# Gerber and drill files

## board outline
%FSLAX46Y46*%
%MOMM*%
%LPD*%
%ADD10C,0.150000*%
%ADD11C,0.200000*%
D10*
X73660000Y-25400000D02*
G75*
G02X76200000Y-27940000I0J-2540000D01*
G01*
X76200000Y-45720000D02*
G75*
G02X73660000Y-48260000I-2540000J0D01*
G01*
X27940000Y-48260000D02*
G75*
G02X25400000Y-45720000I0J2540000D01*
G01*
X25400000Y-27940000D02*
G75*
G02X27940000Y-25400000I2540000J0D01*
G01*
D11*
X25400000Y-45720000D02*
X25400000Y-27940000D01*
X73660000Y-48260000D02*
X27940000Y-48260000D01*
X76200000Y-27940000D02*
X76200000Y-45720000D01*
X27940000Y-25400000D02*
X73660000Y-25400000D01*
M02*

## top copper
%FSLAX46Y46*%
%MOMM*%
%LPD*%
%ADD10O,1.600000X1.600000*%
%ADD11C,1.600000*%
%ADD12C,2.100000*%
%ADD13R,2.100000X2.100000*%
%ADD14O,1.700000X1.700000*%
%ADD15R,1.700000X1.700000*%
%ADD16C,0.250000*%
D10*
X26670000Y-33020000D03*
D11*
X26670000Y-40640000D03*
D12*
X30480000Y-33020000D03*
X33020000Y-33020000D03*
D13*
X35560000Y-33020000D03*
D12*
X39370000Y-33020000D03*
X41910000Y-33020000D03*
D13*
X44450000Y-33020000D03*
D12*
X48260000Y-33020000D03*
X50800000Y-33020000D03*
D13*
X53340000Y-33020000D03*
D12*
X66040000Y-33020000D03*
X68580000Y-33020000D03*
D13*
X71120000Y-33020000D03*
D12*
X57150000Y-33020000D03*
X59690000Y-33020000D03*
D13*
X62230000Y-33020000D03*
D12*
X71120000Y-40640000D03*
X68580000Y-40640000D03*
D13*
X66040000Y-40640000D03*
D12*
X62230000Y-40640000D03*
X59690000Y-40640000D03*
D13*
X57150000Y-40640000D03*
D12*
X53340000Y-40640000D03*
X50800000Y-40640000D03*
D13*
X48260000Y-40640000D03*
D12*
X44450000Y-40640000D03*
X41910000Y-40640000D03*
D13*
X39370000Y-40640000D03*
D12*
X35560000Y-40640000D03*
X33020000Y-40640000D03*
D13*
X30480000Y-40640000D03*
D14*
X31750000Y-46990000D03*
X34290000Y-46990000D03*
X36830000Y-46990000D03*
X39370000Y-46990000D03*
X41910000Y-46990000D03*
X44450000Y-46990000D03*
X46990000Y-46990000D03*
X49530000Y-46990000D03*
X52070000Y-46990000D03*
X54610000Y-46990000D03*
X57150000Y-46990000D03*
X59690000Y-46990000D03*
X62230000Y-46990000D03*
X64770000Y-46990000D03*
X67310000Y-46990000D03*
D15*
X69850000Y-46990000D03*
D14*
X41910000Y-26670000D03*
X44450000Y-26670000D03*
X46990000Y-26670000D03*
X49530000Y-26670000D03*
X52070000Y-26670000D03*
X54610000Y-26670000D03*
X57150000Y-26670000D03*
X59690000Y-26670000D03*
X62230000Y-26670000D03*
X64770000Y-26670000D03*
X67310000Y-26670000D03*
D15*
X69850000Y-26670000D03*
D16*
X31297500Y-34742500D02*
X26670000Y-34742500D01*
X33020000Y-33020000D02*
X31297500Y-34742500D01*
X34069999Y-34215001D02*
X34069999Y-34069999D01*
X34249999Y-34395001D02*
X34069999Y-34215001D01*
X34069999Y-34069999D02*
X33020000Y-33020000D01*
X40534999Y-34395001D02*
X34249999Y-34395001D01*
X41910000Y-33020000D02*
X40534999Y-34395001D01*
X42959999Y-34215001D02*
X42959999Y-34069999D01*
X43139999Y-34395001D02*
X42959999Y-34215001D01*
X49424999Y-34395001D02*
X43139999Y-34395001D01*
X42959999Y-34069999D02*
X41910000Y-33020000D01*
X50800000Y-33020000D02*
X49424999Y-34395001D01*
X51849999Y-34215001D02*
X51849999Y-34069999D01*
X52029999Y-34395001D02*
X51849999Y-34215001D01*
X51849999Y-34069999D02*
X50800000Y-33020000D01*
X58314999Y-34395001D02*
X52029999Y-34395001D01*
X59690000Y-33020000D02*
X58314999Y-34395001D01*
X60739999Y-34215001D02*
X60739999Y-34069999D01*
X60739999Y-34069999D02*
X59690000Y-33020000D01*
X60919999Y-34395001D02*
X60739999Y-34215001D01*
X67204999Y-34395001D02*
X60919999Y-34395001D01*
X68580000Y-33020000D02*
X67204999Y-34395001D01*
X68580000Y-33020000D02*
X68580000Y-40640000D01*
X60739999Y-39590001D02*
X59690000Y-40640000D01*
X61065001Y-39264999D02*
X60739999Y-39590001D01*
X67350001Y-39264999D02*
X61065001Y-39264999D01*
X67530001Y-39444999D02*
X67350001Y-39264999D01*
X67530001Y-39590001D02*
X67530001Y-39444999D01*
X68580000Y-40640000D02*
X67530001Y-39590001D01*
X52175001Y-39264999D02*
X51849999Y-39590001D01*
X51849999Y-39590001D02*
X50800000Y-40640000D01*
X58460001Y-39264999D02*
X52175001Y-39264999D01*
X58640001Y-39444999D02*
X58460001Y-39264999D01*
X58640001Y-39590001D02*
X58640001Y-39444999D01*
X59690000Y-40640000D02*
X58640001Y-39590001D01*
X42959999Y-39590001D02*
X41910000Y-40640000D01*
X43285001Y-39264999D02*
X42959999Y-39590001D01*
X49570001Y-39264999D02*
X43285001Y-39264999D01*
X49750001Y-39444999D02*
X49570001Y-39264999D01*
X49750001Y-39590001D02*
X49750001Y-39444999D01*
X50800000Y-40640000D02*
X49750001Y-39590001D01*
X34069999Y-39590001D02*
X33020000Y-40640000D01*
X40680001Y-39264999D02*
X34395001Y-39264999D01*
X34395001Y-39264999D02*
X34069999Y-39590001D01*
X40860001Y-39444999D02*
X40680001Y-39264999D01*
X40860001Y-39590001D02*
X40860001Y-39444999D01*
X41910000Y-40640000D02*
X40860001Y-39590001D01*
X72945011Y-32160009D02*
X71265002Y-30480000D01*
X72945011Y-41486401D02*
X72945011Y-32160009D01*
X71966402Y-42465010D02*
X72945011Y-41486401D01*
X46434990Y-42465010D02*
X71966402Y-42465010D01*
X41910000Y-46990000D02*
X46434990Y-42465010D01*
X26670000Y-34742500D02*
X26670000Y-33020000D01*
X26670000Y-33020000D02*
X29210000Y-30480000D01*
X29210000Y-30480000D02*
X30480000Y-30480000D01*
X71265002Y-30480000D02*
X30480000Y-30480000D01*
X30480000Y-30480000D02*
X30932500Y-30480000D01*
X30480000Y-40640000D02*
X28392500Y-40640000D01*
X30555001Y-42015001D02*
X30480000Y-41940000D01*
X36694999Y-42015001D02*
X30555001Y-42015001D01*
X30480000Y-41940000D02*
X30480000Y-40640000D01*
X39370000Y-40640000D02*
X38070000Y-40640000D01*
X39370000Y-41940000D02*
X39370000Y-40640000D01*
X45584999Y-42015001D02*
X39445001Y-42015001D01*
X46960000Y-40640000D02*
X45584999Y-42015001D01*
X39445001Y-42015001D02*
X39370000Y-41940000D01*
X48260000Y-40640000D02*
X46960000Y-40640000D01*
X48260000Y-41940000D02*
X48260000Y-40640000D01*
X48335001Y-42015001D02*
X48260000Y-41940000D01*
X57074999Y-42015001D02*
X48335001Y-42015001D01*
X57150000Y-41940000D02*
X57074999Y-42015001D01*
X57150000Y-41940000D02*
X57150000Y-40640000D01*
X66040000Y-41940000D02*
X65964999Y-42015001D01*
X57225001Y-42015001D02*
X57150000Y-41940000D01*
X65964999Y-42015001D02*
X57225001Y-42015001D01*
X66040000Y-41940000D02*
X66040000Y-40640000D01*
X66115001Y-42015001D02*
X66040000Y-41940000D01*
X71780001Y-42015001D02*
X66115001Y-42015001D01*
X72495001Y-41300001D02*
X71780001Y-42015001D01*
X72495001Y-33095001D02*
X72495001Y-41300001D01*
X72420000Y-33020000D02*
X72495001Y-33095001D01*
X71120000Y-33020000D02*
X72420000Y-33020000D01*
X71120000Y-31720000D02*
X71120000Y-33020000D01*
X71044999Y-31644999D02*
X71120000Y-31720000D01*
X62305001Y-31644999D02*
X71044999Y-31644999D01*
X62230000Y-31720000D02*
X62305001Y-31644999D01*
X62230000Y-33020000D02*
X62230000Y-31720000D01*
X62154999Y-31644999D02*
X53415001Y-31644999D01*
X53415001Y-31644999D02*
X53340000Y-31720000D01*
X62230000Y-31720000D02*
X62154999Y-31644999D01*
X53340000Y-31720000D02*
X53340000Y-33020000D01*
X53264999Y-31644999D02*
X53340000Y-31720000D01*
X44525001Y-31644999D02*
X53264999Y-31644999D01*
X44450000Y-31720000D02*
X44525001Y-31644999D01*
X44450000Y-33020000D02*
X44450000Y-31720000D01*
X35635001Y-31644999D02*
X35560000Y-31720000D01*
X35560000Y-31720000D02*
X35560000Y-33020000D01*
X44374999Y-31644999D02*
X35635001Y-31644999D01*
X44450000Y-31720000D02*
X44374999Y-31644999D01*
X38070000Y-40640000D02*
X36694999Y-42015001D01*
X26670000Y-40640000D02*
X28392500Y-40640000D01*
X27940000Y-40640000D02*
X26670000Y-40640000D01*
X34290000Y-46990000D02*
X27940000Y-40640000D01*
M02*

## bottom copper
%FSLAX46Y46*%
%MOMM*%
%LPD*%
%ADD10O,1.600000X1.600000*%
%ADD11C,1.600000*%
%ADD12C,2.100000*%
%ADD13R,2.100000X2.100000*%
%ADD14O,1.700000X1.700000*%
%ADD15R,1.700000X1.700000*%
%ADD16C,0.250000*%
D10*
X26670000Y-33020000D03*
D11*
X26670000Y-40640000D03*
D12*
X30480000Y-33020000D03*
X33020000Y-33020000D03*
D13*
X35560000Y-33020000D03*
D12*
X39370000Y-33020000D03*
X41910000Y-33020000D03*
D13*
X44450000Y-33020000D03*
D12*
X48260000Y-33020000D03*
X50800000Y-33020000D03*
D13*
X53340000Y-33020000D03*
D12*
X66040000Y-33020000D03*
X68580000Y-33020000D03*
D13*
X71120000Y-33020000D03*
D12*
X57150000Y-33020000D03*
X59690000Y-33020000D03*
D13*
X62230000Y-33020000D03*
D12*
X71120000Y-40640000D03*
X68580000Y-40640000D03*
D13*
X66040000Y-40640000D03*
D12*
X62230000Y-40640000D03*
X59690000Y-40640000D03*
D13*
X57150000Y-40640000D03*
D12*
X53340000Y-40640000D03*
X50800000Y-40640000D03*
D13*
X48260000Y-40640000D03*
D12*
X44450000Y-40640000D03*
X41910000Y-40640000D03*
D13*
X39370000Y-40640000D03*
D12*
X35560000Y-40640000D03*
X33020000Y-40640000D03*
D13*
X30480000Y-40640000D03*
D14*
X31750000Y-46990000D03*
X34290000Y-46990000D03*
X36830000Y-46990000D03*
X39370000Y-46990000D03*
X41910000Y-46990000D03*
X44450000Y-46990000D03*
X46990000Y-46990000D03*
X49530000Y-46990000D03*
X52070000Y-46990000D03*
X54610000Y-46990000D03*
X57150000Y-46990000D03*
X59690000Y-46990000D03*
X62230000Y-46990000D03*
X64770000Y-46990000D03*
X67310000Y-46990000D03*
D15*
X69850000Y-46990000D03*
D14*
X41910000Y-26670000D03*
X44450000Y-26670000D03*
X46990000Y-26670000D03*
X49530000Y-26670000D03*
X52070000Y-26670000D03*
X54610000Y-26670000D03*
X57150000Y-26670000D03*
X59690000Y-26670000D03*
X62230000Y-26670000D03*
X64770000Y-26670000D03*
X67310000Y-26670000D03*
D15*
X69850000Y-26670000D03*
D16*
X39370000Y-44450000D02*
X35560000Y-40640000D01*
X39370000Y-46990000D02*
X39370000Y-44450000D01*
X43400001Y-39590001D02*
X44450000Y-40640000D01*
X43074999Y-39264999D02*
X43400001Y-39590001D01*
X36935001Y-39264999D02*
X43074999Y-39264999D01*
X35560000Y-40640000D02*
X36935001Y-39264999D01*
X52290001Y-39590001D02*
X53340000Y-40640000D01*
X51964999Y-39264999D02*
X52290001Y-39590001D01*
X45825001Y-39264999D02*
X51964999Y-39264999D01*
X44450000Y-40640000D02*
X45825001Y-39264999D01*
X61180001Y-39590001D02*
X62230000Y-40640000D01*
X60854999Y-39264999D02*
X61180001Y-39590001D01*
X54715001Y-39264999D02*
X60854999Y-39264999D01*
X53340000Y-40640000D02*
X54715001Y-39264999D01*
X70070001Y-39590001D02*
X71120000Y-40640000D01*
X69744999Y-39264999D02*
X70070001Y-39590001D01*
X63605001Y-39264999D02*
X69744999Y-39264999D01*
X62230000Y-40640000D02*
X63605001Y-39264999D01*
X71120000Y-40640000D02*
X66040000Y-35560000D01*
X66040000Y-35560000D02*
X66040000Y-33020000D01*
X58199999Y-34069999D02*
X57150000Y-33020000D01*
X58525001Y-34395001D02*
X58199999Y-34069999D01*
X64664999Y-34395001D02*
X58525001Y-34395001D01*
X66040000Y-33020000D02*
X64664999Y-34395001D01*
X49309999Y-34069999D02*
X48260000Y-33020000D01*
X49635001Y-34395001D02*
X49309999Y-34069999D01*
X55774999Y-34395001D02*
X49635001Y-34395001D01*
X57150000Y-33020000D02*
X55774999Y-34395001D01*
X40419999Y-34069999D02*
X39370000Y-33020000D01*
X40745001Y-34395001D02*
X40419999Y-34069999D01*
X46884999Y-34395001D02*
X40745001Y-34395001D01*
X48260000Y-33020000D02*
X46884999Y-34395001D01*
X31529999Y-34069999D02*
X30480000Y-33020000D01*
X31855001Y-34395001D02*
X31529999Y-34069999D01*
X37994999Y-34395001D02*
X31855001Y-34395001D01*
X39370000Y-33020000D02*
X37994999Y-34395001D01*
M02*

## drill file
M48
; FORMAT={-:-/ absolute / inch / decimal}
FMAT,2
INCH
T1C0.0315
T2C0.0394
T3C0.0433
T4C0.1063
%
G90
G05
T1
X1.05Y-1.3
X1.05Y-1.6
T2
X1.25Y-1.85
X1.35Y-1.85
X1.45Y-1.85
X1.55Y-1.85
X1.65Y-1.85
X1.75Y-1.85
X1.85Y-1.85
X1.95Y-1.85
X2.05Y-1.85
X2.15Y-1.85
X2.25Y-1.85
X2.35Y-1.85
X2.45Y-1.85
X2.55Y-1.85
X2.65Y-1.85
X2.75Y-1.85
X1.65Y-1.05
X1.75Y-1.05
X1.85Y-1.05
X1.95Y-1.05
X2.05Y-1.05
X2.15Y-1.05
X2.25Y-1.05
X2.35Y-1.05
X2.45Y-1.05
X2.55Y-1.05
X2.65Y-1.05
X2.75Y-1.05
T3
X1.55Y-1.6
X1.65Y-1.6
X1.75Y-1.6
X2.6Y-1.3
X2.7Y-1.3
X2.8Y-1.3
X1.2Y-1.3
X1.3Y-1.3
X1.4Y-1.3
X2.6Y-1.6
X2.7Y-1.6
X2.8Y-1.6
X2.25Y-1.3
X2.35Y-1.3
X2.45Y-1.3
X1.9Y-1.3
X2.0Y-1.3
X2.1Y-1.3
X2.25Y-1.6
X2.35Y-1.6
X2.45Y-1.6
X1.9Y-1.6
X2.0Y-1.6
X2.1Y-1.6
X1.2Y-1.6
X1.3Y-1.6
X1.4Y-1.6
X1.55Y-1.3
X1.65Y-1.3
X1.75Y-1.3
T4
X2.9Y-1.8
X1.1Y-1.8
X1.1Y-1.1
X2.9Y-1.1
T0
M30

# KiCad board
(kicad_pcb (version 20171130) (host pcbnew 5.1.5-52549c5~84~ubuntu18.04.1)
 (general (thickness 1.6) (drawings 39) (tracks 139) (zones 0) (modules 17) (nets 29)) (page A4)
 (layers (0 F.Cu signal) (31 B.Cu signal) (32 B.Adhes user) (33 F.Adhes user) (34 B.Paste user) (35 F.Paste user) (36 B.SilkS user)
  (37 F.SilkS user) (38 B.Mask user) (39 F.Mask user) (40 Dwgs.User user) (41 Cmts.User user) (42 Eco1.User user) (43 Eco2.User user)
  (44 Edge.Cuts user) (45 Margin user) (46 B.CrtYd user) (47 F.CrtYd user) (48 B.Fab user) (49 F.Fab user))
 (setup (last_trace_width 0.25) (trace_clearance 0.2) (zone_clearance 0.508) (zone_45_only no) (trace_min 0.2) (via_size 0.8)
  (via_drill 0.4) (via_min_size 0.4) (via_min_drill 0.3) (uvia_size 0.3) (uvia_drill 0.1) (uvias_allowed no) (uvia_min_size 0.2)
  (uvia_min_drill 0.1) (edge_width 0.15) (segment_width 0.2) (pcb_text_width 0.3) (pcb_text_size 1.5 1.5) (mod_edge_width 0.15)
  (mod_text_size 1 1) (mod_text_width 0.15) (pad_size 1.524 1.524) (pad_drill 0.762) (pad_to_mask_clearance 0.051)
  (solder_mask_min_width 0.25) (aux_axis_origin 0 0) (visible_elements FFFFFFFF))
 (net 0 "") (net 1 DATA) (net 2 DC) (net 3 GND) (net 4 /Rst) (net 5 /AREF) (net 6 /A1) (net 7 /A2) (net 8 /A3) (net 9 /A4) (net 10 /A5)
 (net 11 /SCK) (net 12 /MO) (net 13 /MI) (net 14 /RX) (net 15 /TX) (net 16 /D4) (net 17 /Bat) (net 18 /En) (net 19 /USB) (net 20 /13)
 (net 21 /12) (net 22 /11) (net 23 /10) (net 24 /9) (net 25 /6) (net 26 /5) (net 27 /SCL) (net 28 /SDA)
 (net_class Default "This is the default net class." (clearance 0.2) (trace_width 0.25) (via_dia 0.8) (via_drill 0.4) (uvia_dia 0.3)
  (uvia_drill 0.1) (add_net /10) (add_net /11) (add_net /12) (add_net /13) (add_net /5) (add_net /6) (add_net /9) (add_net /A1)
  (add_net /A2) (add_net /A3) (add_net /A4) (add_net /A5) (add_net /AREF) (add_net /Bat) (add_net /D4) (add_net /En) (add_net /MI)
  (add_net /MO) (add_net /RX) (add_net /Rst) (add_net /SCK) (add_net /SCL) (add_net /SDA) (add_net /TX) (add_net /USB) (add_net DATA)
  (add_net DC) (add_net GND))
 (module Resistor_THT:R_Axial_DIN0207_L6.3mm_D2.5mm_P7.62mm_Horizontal (layer F.Cu) (at 26.67 40.64 90)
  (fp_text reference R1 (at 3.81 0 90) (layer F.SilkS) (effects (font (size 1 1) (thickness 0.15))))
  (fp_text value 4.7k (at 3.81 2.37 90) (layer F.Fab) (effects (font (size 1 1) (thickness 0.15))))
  (pad 2 thru_hole oval (at 7.62 0 90) (size 1.6 1.6) (drill 0.8) (layers *.Cu *.Mask) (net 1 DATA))
  (pad 1 thru_hole circle (at 0 0 90) (size 1.6 1.6) (drill 0.8) (layers *.Cu *.Mask) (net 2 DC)))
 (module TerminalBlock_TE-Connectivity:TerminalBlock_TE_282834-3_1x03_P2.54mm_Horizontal (layer F.Cu) (at 35.56 33.02 180)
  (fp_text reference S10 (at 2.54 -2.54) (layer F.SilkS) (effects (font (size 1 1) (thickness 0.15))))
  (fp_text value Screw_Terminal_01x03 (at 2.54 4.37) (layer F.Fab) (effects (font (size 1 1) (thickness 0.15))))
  (pad 3 thru_hole circle (at 5.08 0 180) (size 2.1 2.1) (drill 1.1) (layers *.Cu *.Mask) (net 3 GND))
  (pad 2 thru_hole circle (at 2.54 0 180) (size 2.1 2.1) (drill 1.1) (layers *.Cu *.Mask) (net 1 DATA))
  (pad 1 thru_hole rect (at 0 0 180) (size 2.1 2.1) (drill 1.1) (layers *.Cu *.Mask) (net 2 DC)))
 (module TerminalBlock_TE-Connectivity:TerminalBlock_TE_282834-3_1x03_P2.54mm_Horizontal (layer F.Cu) (at 44.45 33.02 180)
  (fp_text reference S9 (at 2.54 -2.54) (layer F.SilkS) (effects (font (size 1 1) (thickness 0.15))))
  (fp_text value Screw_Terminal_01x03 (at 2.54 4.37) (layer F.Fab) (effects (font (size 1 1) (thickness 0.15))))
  (pad 3 thru_hole circle (at 5.08 0 180) (size 2.1 2.1) (drill 1.1) (layers *.Cu *.Mask) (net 3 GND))
  (pad 2 thru_hole circle (at 2.54 0 180) (size 2.1 2.1) (drill 1.1) (layers *.Cu *.Mask) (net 1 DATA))
  (pad 1 thru_hole rect (at 0 0 180) (size 2.1 2.1) (drill 1.1) (layers *.Cu *.Mask) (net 2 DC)))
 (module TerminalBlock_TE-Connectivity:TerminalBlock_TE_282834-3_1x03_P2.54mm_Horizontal (layer F.Cu) (at 53.34 33.02 180)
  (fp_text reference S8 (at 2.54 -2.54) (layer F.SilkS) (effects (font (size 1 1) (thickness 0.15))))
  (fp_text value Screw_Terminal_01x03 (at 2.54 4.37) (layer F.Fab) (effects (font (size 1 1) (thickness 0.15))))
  (pad 3 thru_hole circle (at 5.08 0 180) (size 2.1 2.1) (drill 1.1) (layers *.Cu *.Mask) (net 3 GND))
  (pad 2 thru_hole circle (at 2.54 0 180) (size 2.1 2.1) (drill 1.1) (layers *.Cu *.Mask) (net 1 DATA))
  (pad 1 thru_hole rect (at 0 0 180) (size 2.1 2.1) (drill 1.1) (layers *.Cu *.Mask) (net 2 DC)))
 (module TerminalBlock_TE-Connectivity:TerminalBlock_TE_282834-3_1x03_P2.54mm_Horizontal (layer F.Cu) (at 71.12 33.02 180)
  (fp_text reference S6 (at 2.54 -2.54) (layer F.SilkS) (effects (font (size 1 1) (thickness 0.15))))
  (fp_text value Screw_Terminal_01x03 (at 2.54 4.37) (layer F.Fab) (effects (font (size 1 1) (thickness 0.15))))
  (pad 3 thru_hole circle (at 5.08 0 180) (size 2.1 2.1) (drill 1.1) (layers *.Cu *.Mask) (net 3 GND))
  (pad 2 thru_hole circle (at 2.54 0 180) (size 2.1 2.1) (drill 1.1) (layers *.Cu *.Mask) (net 1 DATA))
  (pad 1 thru_hole rect (at 0 0 180) (size 2.1 2.1) (drill 1.1) (layers *.Cu *.Mask) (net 2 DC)))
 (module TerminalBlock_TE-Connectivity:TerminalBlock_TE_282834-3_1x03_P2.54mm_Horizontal (layer F.Cu) (at 62.23 33.02 180)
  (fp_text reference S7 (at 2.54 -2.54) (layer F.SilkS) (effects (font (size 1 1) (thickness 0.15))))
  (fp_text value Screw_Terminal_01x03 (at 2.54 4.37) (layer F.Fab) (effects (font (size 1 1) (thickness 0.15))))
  (pad 3 thru_hole circle (at 5.08 0 180) (size 2.1 2.1) (drill 1.1) (layers *.Cu *.Mask) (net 3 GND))
  (pad 2 thru_hole circle (at 2.54 0 180) (size 2.1 2.1) (drill 1.1) (layers *.Cu *.Mask) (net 1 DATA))
  (pad 1 thru_hole rect (at 0 0 180) (size 2.1 2.1) (drill 1.1) (layers *.Cu *.Mask) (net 2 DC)))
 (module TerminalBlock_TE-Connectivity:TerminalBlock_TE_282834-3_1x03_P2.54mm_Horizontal (layer F.Cu) (at 66.04 40.64)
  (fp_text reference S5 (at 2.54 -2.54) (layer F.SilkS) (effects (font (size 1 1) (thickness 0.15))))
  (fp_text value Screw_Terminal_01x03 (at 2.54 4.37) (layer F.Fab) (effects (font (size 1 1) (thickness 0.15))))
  (pad 3 thru_hole circle (at 5.08 0) (size 2.1 2.1) (drill 1.1) (layers *.Cu *.Mask) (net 3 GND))
  (pad 2 thru_hole circle (at 2.54 0) (size 2.1 2.1) (drill 1.1) (layers *.Cu *.Mask) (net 1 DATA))
  (pad 1 thru_hole rect (at 0 0) (size 2.1 2.1) (drill 1.1) (layers *.Cu *.Mask) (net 2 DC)))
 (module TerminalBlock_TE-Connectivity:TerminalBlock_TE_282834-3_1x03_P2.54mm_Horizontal (layer F.Cu) (at 57.15 40.64)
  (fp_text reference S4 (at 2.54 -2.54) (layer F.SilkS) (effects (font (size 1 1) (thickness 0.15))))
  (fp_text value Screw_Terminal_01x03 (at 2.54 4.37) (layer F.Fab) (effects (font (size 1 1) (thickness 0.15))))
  (pad 3 thru_hole circle (at 5.08 0) (size 2.1 2.1) (drill 1.1) (layers *.Cu *.Mask) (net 3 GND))
  (pad 2 thru_hole circle (at 2.54 0) (size 2.1 2.1) (drill 1.1) (layers *.Cu *.Mask) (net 1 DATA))
  (pad 1 thru_hole rect (at 0 0) (size 2.1 2.1) (drill 1.1) (layers *.Cu *.Mask) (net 2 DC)))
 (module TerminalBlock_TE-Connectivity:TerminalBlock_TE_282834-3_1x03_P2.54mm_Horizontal (layer F.Cu) (at 48.26 40.64)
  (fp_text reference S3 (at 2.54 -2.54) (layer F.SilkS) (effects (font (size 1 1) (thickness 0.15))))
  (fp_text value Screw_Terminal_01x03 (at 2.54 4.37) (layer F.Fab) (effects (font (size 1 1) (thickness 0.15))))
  (pad 3 thru_hole circle (at 5.08 0) (size 2.1 2.1) (drill 1.1) (layers *.Cu *.Mask) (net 3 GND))
  (pad 2 thru_hole circle (at 2.54 0) (size 2.1 2.1) (drill 1.1) (layers *.Cu *.Mask) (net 1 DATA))
  (pad 1 thru_hole rect (at 0 0) (size 2.1 2.1) (drill 1.1) (layers *.Cu *.Mask) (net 2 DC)))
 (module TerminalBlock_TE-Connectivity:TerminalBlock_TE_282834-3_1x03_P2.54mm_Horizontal (layer F.Cu) (at 39.37 40.64)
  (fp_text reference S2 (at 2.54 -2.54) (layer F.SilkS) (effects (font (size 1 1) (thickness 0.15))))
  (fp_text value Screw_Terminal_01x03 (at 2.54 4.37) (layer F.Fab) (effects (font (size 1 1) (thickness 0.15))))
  (pad 3 thru_hole circle (at 5.08 0) (size 2.1 2.1) (drill 1.1) (layers *.Cu *.Mask) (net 3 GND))
  (pad 2 thru_hole circle (at 2.54 0) (size 2.1 2.1) (drill 1.1) (layers *.Cu *.Mask) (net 1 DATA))
  (pad 1 thru_hole rect (at 0 0) (size 2.1 2.1) (drill 1.1) (layers *.Cu *.Mask) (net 2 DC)))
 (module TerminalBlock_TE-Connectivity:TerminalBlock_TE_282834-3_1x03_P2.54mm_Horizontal (layer F.Cu) (at 30.48 40.64)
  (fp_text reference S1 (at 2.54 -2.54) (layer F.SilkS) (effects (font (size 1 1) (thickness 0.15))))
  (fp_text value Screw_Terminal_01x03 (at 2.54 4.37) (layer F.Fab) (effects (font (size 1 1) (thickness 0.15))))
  (pad 3 thru_hole circle (at 5.08 0) (size 2.1 2.1) (drill 1.1) (layers *.Cu *.Mask) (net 3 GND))
  (pad 2 thru_hole circle (at 2.54 0) (size 2.1 2.1) (drill 1.1) (layers *.Cu *.Mask) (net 1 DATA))
  (pad 1 thru_hole rect (at 0 0) (size 2.1 2.1) (drill 1.1) (layers *.Cu *.Mask) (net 2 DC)))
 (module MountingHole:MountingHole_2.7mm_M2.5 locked (layer F.Cu) (at 73.66 27.94)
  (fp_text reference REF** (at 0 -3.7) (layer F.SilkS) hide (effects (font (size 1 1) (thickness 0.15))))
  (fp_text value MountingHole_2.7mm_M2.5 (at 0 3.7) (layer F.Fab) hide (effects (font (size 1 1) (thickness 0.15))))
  (pad 1 np_thru_hole circle (at 0 0) (size 2.7 2.7) (drill 2.7) (layers *.Cu *.Mask)))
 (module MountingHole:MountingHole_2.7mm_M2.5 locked (layer F.Cu) (at 73.66 45.72)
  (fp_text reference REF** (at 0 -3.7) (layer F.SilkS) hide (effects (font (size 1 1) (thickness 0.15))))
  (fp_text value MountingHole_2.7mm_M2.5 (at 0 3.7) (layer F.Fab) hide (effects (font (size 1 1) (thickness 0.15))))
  (pad 1 np_thru_hole circle (at 0 0) (size 2.7 2.7) (drill 2.7) (layers *.Cu *.Mask)))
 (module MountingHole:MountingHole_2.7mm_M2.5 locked (layer F.Cu) (at 27.94 45.72)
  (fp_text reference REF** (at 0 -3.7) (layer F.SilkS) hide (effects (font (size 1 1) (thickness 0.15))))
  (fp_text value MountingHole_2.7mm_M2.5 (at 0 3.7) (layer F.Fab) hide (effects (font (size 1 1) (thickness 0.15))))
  (pad 1 np_thru_hole circle (at 0 0) (size 2.7 2.7) (drill 2.7) (layers *.Cu *.Mask)))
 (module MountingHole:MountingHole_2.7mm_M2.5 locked (layer F.Cu) (at 27.94 27.94)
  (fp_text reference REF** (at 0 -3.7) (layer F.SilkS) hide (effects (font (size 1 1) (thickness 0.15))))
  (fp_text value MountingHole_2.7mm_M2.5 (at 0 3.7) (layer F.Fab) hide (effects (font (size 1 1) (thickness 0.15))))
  (pad 1 np_thru_hole circle (at 0 0) (size 2.7 2.7) (drill 2.7) (layers *.Cu *.Mask)))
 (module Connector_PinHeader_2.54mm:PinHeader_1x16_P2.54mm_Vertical (layer B.Cu) (at 69.85 46.99 90)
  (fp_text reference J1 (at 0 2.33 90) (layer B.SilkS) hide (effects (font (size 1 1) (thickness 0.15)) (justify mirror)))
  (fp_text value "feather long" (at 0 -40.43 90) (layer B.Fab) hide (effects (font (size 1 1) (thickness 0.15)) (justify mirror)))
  (pad 16 thru_hole oval (at 0 -38.1 90) (size 1.7 1.7) (drill 1) (layers *.Cu *.Mask) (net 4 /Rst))
  (pad 15 thru_hole oval (at 0 -35.56 90) (size 1.7 1.7) (drill 1) (layers *.Cu *.Mask) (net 2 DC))
  (pad 14 thru_hole oval (at 0 -33.02 90) (size 1.7 1.7) (drill 1) (layers *.Cu *.Mask) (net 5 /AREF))
  (pad 13 thru_hole oval (at 0 -30.48 90) (size 1.7 1.7) (drill 1) (layers *.Cu *.Mask) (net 3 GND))
  (pad 12 thru_hole oval (at 0 -27.94 90) (size 1.7 1.7) (drill 1) (layers *.Cu *.Mask) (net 1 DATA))
  (pad 11 thru_hole oval (at 0 -25.4 90) (size 1.7 1.7) (drill 1) (layers *.Cu *.Mask) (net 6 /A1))
  (pad 10 thru_hole oval (at 0 -22.86 90) (size 1.7 1.7) (drill 1) (layers *.Cu *.Mask) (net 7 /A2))
  (pad 9 thru_hole oval (at 0 -20.32 90) (size 1.7 1.7) (drill 1) (layers *.Cu *.Mask) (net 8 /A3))
  (pad 8 thru_hole oval (at 0 -17.78 90) (size 1.7 1.7) (drill 1) (layers *.Cu *.Mask) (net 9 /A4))
  (pad 7 thru_hole oval (at 0 -15.24 90) (size 1.7 1.7) (drill 1) (layers *.Cu *.Mask) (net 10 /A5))
  (pad 6 thru_hole oval (at 0 -12.7 90) (size 1.7 1.7) (drill 1) (layers *.Cu *.Mask) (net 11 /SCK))
  (pad 5 thru_hole oval (at 0 -10.16 90) (size 1.7 1.7) (drill 1) (layers *.Cu *.Mask) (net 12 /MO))
  (pad 4 thru_hole oval (at 0 -7.62 90) (size 1.7 1.7) (drill 1) (layers *.Cu *.Mask) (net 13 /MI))
  (pad 3 thru_hole oval (at 0 -5.08 90) (size 1.7 1.7) (drill 1) (layers *.Cu *.Mask) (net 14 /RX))
  (pad 2 thru_hole oval (at 0 -2.54 90) (size 1.7 1.7) (drill 1) (layers *.Cu *.Mask) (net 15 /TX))
  (pad 1 thru_hole rect (at 0 0 90) (size 1.7 1.7) (drill 1) (layers *.Cu *.Mask) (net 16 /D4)))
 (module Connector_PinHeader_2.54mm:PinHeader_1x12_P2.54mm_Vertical (layer B.Cu) (at 69.85 26.67 90)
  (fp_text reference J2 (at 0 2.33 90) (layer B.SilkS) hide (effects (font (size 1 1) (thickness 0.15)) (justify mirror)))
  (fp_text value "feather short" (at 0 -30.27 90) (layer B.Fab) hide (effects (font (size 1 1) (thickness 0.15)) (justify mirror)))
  (pad 12 thru_hole oval (at 0 -27.94 90) (size 1.7 1.7) (drill 1) (layers *.Cu *.Mask) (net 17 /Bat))
  (pad 11 thru_hole oval (at 0 -25.4 90) (size 1.7 1.7) (drill 1) (layers *.Cu *.Mask) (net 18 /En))
  (pad 10 thru_hole oval (at 0 -22.86 90) (size 1.7 1.7) (drill 1) (layers *.Cu *.Mask) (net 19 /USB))
  (pad 9 thru_hole oval (at 0 -20.32 90) (size 1.7 1.7) (drill 1) (layers *.Cu *.Mask) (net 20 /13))
  (pad 8 thru_hole oval (at 0 -17.78 90) (size 1.7 1.7) (drill 1) (layers *.Cu *.Mask) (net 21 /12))
  (pad 7 thru_hole oval (at 0 -15.24 90) (size 1.7 1.7) (drill 1) (layers *.Cu *.Mask) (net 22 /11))
  (pad 6 thru_hole oval (at 0 -12.7 90) (size 1.7 1.7) (drill 1) (layers *.Cu *.Mask) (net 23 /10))
  (pad 5 thru_hole oval (at 0 -10.16 90) (size 1.7 1.7) (drill 1) (layers *.Cu *.Mask) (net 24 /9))
  (pad 4 thru_hole oval (at 0 -7.62 90) (size 1.7 1.7) (drill 1) (layers *.Cu *.Mask) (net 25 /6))
  (pad 3 thru_hole oval (at 0 -5.08 90) (size 1.7 1.7) (drill 1) (layers *.Cu *.Mask) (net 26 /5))
  (pad 2 thru_hole oval (at 0 -2.54 90) (size 1.7 1.7) (drill 1) (layers *.Cu *.Mask) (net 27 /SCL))
  (pad 1 thru_hole rect (at 0 0 90) (size 1.7 1.7) (drill 1) (layers *.Cu *.Mask) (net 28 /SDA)))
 (gr_arc (start 73.66 27.94) (end 76.2 27.94) (angle -90) (layer Edge.Cuts) (width 0.15))
 (gr_arc (start 73.66 45.72) (end 73.66 48.26) (angle -90) (layer Edge.Cuts) (width 0.15))
 (gr_arc (start 27.94 45.72) (end 25.4 45.72) (angle -90) (layer Edge.Cuts) (width 0.15))
 (gr_arc (start 27.94 27.94) (end 27.94 25.4) (angle -90) (layer Edge.Cuts) (width 0.15))
 (gr_line (start 25.4 45.72) (end 25.4 27.94) (layer Edge.Cuts) (width 0.2))
 (gr_line (start 73.66 48.26) (end 27.94 48.26) (layer Edge.Cuts) (width 0.2))
 (gr_line (start 76.2 27.94) (end 76.2 45.72) (layer Edge.Cuts) (width 0.2))
 (gr_line (start 27.94 25.4) (end 73.66 25.4) (layer Edge.Cuts) (width 0.2))
 (segment (start 39.37 44.45) (end 35.56 40.64) (width 0.25) (layer B.Cu) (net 3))
 (segment (start 39.37 46.99) (end 39.37 44.45) (width 0.25) (layer B.Cu) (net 3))
 (segment (start 43.400001 39.590001) (end 44.45 40.64) (width 0.25) (layer B.Cu) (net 3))
 (segment (start 43.074999 39.264999) (end 43.400001 39.590001) (width 0.25) (layer B.Cu) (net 3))
 (segment (start 36.935001 39.264999) (end 43.074999 39.264999) (width 0.25) (layer B.Cu) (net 3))
 (segment (start 35.56 40.64) (end 36.935001 39.264999) (width 0.25) (layer B.Cu) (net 3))
 (segment (start 52.290001 39.590001) (end 53.34 40.64) (width 0.25) (layer B.Cu) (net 3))
 (segment (start 51.964999 39.264999) (end 52.290001 39.590001) (width 0.25) (layer B.Cu) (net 3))
 (segment (start 45.825001 39.264999) (end 51.964999 39.264999) (width 0.25) (layer B.Cu) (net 3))
 (segment (start 44.45 40.64) (end 45.825001 39.264999) (width 0.25) (layer B.Cu) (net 3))
 (segment (start 61.180001 39.590001) (end 62.23 40.64) (width 0.25) (layer B.Cu) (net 3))
 (segment (start 60.854999 39.264999) (end 61.180001 39.590001) (width 0.25) (layer B.Cu) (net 3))
 (segment (start 54.715001 39.264999) (end 60.854999 39.264999) (width 0.25) (layer B.Cu) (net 3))
 (segment (start 53.34 40.64) (end 54.715001 39.264999) (width 0.25) (layer B.Cu) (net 3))
 (segment (start 70.070001 39.590001) (end 71.12 40.64) (width 0.25) (layer B.Cu) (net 3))
 (segment (start 69.744999 39.264999) (end 70.070001 39.590001) (width 0.25) (layer B.Cu) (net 3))
 (segment (start 63.605001 39.264999) (end 69.744999 39.264999) (width 0.25) (layer B.Cu) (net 3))
 (segment (start 62.23 40.64) (end 63.605001 39.264999) (width 0.25) (layer B.Cu) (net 3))
 (segment (start 71.12 40.64) (end 66.04 35.56) (width 0.25) (layer B.Cu) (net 3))
 (segment (start 66.04 35.56) (end 66.04 33.02) (width 0.25) (layer B.Cu) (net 3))
 (segment (start 58.199999 34.069999) (end 57.15 33.02) (width 0.25) (layer B.Cu) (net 3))
 (segment (start 58.525001 34.395001) (end 58.199999 34.069999) (width 0.25) (layer B.Cu) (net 3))
 (segment (start 64.664999 34.395001) (end 58.525001 34.395001) (width 0.25) (layer B.Cu) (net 3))
 (segment (start 66.04 33.02) (end 64.664999 34.395001) (width 0.25) (layer B.Cu) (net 3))
 (segment (start 49.309999 34.069999) (end 48.26 33.02) (width 0.25) (layer B.Cu) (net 3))
 (segment (start 49.635001 34.395001) (end 49.309999 34.069999) (width 0.25) (layer B.Cu) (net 3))
 (segment (start 55.774999 34.395001) (end 49.635001 34.395001) (width 0.25) (layer B.Cu) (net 3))
 (segment (start 57.15 33.02) (end 55.774999 34.395001) (width 0.25) (layer B.Cu) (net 3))
 (segment (start 40.419999 34.069999) (end 39.37 33.02) (width 0.25) (layer B.Cu) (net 3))
 (segment (start 40.745001 34.395001) (end 40.419999 34.069999) (width 0.25) (layer B.Cu) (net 3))
 (segment (start 46.884999 34.395001) (end 40.745001 34.395001) (width 0.25) (layer B.Cu) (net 3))
 (segment (start 48.26 33.02) (end 46.884999 34.395001) (width 0.25) (layer B.Cu) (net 3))
 (segment (start 31.529999 34.069999) (end 30.48 33.02) (width 0.25) (layer B.Cu) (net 3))
 (segment (start 31.855001 34.395001) (end 31.529999 34.069999) (width 0.25) (layer B.Cu) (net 3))
 (segment (start 37.994999 34.395001) (end 31.855001 34.395001) (width 0.25) (layer B.Cu) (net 3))
 (segment (start 39.37 33.02) (end 37.994999 34.395001) (width 0.25) (layer B.Cu) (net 3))
 (segment (start 31.2975 34.7425) (end 26.67 34.7425) (width 0.25) (layer F.Cu) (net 1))
 (segment (start 33.02 33.02) (end 31.2975 34.7425) (width 0.25) (layer F.Cu) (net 1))
 (segment (start 34.069999 34.215001) (end 34.069999 34.069999) (width 0.25) (layer F.Cu) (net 1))
 (segment (start 34.249999 34.395001) (end 34.069999 34.215001) (width 0.25) (layer F.Cu) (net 1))
 (segment (start 34.069999 34.069999) (end 33.02 33.02) (width 0.25) (layer F.Cu) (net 1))
 (segment (start 40.534999 34.395001) (end 34.249999 34.395001) (width 0.25) (layer F.Cu) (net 1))
 (segment (start 41.91 33.02) (end 40.534999 34.395001) (width 0.25) (layer F.Cu) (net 1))
 (segment (start 42.959999 34.215001) (end 42.959999 34.069999) (width 0.25) (layer F.Cu) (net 1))
 (segment (start 43.139999 34.395001) (end 42.959999 34.215001) (width 0.25) (layer F.Cu) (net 1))
 (segment (start 49.424999 34.395001) (end 43.139999 34.395001) (width 0.25) (layer F.Cu) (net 1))
 (segment (start 42.959999 34.069999) (end 41.91 33.02) (width 0.25) (layer F.Cu) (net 1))
 (segment (start 50.8 33.02) (end 49.424999 34.395001) (width 0.25) (layer F.Cu) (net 1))
 (segment (start 51.849999 34.215001) (end 51.849999 34.069999) (width 0.25) (layer F.Cu) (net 1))
 (segment (start 52.029999 34.395001) (end 51.849999 34.215001) (width 0.25) (layer F.Cu) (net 1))
 (segment (start 51.849999 34.069999) (end 50.8 33.02) (width 0.25) (layer F.Cu) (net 1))
 (segment (start 58.314999 34.395001) (end 52.029999 34.395001) (width 0.25) (layer F.Cu) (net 1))
 (segment (start 59.69 33.02) (end 58.314999 34.395001) (width 0.25) (layer F.Cu) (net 1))
 (segment (start 60.739999 34.215001) (end 60.739999 34.069999) (width 0.25) (layer F.Cu) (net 1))
 (segment (start 60.739999 34.069999) (end 59.69 33.02) (width 0.25) (layer F.Cu) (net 1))
 (segment (start 60.919999 34.395001) (end 60.739999 34.215001) (width 0.25) (layer F.Cu) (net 1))
 (segment (start 67.204999 34.395001) (end 60.919999 34.395001) (width 0.25) (layer F.Cu) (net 1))
 (segment (start 68.58 33.02) (end 67.204999 34.395001) (width 0.25) (layer F.Cu) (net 1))
 (segment (start 68.58 33.02) (end 68.58 40.64) (width 0.25) (layer F.Cu) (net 1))
 (segment (start 60.739999 39.590001) (end 59.69 40.64) (width 0.25) (layer F.Cu) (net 1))
 (segment (start 61.065001 39.264999) (end 60.739999 39.590001) (width 0.25) (layer F.Cu) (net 1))
 (segment (start 67.350001 39.264999) (end 61.065001 39.264999) (width 0.25) (layer F.Cu) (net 1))
 (segment (start 67.530001 39.444999) (end 67.350001 39.264999) (width 0.25) (layer F.Cu) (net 1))
 (segment (start 67.530001 39.590001) (end 67.530001 39.444999) (width 0.25) (layer F.Cu) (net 1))
 (segment (start 68.58 40.64) (end 67.530001 39.590001) (width 0.25) (layer F.Cu) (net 1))
 (segment (start 52.175001 39.264999) (end 51.849999 39.590001) (width 0.25) (layer F.Cu) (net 1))
 (segment (start 51.849999 39.590001) (end 50.8 40.64) (width 0.25) (layer F.Cu) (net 1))
 (segment (start 58.460001 39.264999) (end 52.175001 39.264999) (width 0.25) (layer F.Cu) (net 1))
 (segment (start 58.640001 39.444999) (end 58.460001 39.264999) (width 0.25) (layer F.Cu) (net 1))
 (segment (start 58.640001 39.590001) (end 58.640001 39.444999) (width 0.25) (layer F.Cu) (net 1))
 (segment (start 59.69 40.64) (end 58.640001 39.590001) (width 0.25) (layer F.Cu) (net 1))
 (segment (start 42.959999 39.590001) (end 41.91 40.64) (width 0.25) (layer F.Cu) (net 1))
 (segment (start 43.285001 39.264999) (end 42.959999 39.590001) (width 0.25) (layer F.Cu) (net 1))
 (segment (start 49.570001 39.264999) (end 43.285001 39.264999) (width 0.25) (layer F.Cu) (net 1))
 (segment (start 49.750001 39.444999) (end 49.570001 39.264999) (width 0.25) (layer F.Cu) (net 1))
 (segment (start 49.750001 39.590001) (end 49.750001 39.444999) (width 0.25) (layer F.Cu) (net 1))
 (segment (start 50.8 40.64) (end 49.750001 39.590001) (width 0.25) (layer F.Cu) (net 1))
 (segment (start 34.069999 39.590001) (end 33.02 40.64) (width 0.25) (layer F.Cu) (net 1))
 (segment (start 40.680001 39.264999) (end 34.395001 39.264999) (width 0.25) (layer F.Cu) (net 1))
 (segment (start 34.395001 39.264999) (end 34.069999 39.590001) (width 0.25) (layer F.Cu) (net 1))
 (segment (start 40.860001 39.444999) (end 40.680001 39.264999) (width 0.25) (layer F.Cu) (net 1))
 (segment (start 40.860001 39.590001) (end 40.860001 39.444999) (width 0.25) (layer F.Cu) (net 1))
 (segment (start 41.91 40.64) (end 40.860001 39.590001) (width 0.25) (layer F.Cu) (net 1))
 (segment (start 72.945011 32.160009) (end 71.265002 30.48) (width 0.25) (layer F.Cu) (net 1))
 (segment (start 72.945011 41.486401) (end 72.945011 32.160009) (width 0.25) (layer F.Cu) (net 1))
 (segment (start 71.966402 42.46501) (end 72.945011 41.486401) (width 0.25) (layer F.Cu) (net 1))
 (segment (start 46.43499 42.46501) (end 71.966402 42.46501) (width 0.25) (layer F.Cu) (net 1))
 (segment (start 41.91 46.99) (end 46.43499 42.46501) (width 0.25) (layer F.Cu) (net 1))
 (segment (start 26.67 34.7425) (end 26.67 33.02) (width 0.25) (layer F.Cu) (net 1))
 (segment (start 26.67 33.02) (end 29.21 30.48) (width 0.25) (layer F.Cu) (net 1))
 (segment (start 29.21 30.48) (end 30.48 30.48) (width 0.25) (layer F.Cu) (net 1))
 (segment (start 71.265002 30.48) (end 30.48 30.48) (width 0.25) (layer F.Cu) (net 1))
 (segment (start 30.48 30.48) (end 30.9325 30.48) (width 0.25) (layer F.Cu) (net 1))
 (segment (start 30.48 40.64) (end 28.3925 40.64) (width 0.25) (layer F.Cu) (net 2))
 (segment (start 30.555001 42.015001) (end 30.48 41.94) (width 0.25) (layer F.Cu) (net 2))
 (segment (start 36.694999 42.015001) (end 30.555001 42.015001) (width 0.25) (layer F.Cu) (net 2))
 (segment (start 30.48 41.94) (end 30.48 40.64) (width 0.25) (layer F.Cu) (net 2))
 (segment (start 39.37 40.64) (end 38.07 40.64) (width 0.25) (layer F.Cu) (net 2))
 (segment (start 39.37 41.94) (end 39.37 40.64) (width 0.25) (layer F.Cu) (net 2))
 (segment (start 45.584999 42.015001) (end 39.445001 42.015001) (width 0.25) (layer F.Cu) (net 2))
 (segment (start 46.96 40.64) (end 45.584999 42.015001) (width 0.25) (layer F.Cu) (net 2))
 (segment (start 39.445001 42.015001) (end 39.37 41.94) (width 0.25) (layer F.Cu) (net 2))
 (segment (start 48.26 40.64) (end 46.96 40.64) (width 0.25) (layer F.Cu) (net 2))
 (segment (start 48.26 41.94) (end 48.26 40.64) (width 0.25) (layer F.Cu) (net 2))
 (segment (start 48.335001 42.015001) (end 48.26 41.94) (width 0.25) (layer F.Cu) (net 2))
 (segment (start 57.074999 42.015001) (end 48.335001 42.015001) (width 0.25) (layer F.Cu) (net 2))
 (segment (start 57.15 41.94) (end 57.074999 42.015001) (width 0.25) (layer F.Cu) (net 2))
 (segment (start 57.15 41.94) (end 57.15 40.64) (width 0.25) (layer F.Cu) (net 2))
 (segment (start 66.04 41.94) (end 65.964999 42.015001) (width 0.25) (layer F.Cu) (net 2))
 (segment (start 57.225001 42.015001) (end 57.15 41.94) (width 0.25) (layer F.Cu) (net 2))
 (segment (start 65.964999 42.015001) (end 57.225001 42.015001) (width 0.25) (layer F.Cu) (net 2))
 (segment (start 66.04 41.94) (end 66.04 40.64) (width 0.25) (layer F.Cu) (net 2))
 (segment (start 66.115001 42.015001) (end 66.04 41.94) (width 0.25) (layer F.Cu) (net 2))
 (segment (start 71.780001 42.015001) (end 66.115001 42.015001) (width 0.25) (layer F.Cu) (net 2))
 (segment (start 72.495001 41.300001) (end 71.780001 42.015001) (width 0.25) (layer F.Cu) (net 2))
 (segment (start 72.495001 33.095001) (end 72.495001 41.300001) (width 0.25) (layer F.Cu) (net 2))
 (segment (start 72.42 33.02) (end 72.495001 33.095001) (width 0.25) (layer F.Cu) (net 2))
 (segment (start 71.12 33.02) (end 72.42 33.02) (width 0.25) (layer F.Cu) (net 2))
 (segment (start 71.12 31.72) (end 71.12 33.02) (width 0.25) (layer F.Cu) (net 2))
 (segment (start 71.044999 31.644999) (end 71.12 31.72) (width 0.25) (layer F.Cu) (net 2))
 (segment (start 62.305001 31.644999) (end 71.044999 31.644999) (width 0.25) (layer F.Cu) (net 2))
 (segment (start 62.23 31.72) (end 62.305001 31.644999) (width 0.25) (layer F.Cu) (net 2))
 (segment (start 62.23 33.02) (end 62.23 31.72) (width 0.25) (layer F.Cu) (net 2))
 (segment (start 62.154999 31.644999) (end 53.415001 31.644999) (width 0.25) (layer F.Cu) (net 2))
 (segment (start 53.415001 31.644999) (end 53.34 31.72) (width 0.25) (layer F.Cu) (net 2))
 (segment (start 62.23 31.72) (end 62.154999 31.644999) (width 0.25) (layer F.Cu) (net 2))
 (segment (start 53.34 31.72) (end 53.34 33.02) (width 0.25) (layer F.Cu) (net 2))
 (segment (start 53.264999 31.644999) (end 53.34 31.72) (width 0.25) (layer F.Cu) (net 2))
 (segment (start 44.525001 31.644999) (end 53.264999 31.644999) (width 0.25) (layer F.Cu) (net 2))
 (segment (start 44.45 31.72) (end 44.525001 31.644999) (width 0.25) (layer F.Cu) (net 2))
 (segment (start 44.45 33.02) (end 44.45 31.72) (width 0.25) (layer F.Cu) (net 2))
 (segment (start 35.635001 31.644999) (end 35.56 31.72) (width 0.25) (layer F.Cu) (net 2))
 (segment (start 35.56 31.72) (end 35.56 33.02) (width 0.25) (layer F.Cu) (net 2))
 (segment (start 44.374999 31.644999) (end 35.635001 31.644999) (width 0.25) (layer F.Cu) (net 2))
 (segment (start 44.45 31.72) (end 44.374999 31.644999) (width 0.25) (layer F.Cu) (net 2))
 (segment (start 38.07 40.64) (end 36.694999 42.015001) (width 0.25) (layer F.Cu) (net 2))
 (segment (start 26.67 40.64) (end 28.3925 40.64) (width 0.25) (layer F.Cu) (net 2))
 (segment (start 27.94 40.64) (end 26.67 40.64) (width 0.25) (layer F.Cu) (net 2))
 (segment (start 34.29 46.99) (end 27.94 40.64) (width 0.25) (layer F.Cu) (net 2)))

